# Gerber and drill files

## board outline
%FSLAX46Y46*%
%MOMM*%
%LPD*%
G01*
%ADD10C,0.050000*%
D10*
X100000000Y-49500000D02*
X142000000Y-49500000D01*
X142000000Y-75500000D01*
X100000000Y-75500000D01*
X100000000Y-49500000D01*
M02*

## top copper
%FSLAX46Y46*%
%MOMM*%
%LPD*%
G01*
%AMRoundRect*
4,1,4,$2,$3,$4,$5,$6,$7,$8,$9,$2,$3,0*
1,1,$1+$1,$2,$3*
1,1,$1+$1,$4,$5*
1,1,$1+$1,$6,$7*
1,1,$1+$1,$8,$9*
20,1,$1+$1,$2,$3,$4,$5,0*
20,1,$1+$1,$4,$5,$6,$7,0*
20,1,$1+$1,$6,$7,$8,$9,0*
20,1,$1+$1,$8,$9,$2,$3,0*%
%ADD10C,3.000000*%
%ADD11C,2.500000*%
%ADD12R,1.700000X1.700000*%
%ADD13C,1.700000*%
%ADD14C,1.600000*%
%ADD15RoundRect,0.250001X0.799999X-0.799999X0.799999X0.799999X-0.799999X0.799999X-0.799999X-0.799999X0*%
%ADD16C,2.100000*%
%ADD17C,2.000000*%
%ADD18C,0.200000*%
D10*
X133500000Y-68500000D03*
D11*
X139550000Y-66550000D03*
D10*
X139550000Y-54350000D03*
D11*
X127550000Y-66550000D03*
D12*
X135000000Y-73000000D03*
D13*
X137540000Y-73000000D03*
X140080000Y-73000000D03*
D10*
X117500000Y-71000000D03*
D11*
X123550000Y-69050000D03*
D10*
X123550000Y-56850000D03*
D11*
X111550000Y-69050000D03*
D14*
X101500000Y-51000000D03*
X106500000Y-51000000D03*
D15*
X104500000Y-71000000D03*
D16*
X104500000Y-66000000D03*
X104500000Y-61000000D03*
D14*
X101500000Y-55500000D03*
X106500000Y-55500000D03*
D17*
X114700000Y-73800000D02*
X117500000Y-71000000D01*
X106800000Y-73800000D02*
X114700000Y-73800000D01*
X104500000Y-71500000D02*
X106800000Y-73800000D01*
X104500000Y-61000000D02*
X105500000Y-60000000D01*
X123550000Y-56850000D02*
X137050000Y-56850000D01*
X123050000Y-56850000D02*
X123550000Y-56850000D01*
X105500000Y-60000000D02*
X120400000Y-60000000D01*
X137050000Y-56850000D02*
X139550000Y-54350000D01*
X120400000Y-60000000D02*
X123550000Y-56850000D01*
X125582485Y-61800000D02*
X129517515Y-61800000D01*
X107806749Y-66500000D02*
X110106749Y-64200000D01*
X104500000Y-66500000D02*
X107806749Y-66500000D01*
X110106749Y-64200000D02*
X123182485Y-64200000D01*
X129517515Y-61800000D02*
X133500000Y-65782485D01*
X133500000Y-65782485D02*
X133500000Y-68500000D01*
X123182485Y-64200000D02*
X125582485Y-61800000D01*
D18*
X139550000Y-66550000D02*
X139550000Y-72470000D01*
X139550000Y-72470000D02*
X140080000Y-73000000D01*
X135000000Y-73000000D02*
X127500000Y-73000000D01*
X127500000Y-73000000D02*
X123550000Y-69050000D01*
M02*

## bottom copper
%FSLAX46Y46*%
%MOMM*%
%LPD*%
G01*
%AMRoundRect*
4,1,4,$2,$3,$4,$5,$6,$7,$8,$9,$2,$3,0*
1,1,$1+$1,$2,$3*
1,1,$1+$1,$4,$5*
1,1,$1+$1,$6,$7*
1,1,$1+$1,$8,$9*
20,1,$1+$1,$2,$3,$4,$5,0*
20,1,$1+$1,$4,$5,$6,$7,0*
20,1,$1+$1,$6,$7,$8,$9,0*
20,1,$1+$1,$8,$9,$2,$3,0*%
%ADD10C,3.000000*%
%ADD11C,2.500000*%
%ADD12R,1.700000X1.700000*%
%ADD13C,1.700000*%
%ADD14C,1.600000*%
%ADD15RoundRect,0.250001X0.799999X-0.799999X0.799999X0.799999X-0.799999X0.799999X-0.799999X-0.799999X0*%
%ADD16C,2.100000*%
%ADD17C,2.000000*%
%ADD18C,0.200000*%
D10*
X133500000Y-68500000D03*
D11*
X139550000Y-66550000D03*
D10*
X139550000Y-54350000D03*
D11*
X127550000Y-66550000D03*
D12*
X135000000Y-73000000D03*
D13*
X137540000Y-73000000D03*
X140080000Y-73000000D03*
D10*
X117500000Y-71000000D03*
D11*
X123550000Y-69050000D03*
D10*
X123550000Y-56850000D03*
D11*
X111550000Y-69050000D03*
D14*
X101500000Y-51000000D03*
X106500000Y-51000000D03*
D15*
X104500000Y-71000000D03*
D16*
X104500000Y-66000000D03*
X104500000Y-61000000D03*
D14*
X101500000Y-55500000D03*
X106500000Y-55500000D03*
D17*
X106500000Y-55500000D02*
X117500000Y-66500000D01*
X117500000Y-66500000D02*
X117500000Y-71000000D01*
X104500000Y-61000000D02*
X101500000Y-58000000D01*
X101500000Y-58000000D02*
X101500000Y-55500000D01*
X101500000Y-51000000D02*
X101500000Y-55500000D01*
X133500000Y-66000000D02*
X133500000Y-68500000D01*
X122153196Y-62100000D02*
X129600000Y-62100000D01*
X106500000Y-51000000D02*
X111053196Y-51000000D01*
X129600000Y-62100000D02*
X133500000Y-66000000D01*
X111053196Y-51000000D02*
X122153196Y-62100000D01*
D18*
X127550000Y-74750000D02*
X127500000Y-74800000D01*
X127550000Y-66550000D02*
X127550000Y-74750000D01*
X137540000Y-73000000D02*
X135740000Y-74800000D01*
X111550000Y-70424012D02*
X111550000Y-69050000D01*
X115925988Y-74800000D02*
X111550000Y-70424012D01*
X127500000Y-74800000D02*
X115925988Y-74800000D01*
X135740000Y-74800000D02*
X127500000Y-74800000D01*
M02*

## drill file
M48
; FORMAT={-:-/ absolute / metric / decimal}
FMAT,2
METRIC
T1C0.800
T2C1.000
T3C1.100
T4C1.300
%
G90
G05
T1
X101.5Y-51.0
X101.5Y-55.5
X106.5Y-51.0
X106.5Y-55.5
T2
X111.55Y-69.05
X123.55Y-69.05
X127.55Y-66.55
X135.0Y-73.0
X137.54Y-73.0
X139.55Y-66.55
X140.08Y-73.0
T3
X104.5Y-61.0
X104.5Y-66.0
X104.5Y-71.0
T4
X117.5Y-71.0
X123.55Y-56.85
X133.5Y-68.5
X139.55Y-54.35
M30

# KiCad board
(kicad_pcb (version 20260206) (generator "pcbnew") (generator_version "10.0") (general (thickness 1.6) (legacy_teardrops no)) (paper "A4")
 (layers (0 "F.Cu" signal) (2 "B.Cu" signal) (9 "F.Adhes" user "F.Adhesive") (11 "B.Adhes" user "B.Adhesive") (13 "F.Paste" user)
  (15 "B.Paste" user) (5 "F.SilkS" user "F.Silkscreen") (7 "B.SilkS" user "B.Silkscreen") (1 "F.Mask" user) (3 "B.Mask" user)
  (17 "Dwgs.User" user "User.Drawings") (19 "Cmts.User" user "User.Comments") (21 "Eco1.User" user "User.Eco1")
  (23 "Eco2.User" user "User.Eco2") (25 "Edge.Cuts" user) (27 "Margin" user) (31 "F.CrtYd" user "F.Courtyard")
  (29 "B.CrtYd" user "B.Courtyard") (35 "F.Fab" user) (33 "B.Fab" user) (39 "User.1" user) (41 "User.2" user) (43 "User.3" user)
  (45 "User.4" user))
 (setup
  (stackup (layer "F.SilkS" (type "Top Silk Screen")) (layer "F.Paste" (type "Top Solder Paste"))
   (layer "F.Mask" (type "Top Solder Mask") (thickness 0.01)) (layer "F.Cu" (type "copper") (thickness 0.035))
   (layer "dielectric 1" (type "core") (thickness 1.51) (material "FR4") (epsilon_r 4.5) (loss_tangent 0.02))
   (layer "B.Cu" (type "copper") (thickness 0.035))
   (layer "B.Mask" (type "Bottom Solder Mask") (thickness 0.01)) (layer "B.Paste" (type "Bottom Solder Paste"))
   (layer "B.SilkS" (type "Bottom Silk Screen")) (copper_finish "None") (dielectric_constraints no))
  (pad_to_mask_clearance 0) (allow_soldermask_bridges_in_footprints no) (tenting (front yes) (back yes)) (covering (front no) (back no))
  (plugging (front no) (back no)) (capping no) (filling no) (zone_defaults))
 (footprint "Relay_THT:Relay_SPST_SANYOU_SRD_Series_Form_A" (layer "F.Cu") (at 133.5 68.5 90)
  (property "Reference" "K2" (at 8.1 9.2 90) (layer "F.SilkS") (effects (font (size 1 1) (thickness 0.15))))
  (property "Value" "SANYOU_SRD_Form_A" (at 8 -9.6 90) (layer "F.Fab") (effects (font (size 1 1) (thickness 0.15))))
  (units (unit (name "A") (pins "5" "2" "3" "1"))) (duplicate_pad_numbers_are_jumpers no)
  (pad "1" thru_hole circle (at 0 0 180) (size 3 3) (drill 1.3) (layers "*.Cu" "*.Mask") (remove_unused_layers no) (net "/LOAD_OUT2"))
  (pad "2" thru_hole circle (at 1.95 6.05 180) (size 2.5 2.5) (drill 1) (layers "*.Cu" "*.Mask") (remove_unused_layers no)
   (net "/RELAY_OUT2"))
  (pad "3" thru_hole circle (at 14.15 6.05 180) (size 3 3) (drill 1.3) (layers "*.Cu" "*.Mask") (remove_unused_layers no)
   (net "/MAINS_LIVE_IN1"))
  (pad "5" thru_hole circle (at 1.95 -5.95 180) (size 2.5 2.5) (drill 1) (layers "*.Cu" "*.Mask") (remove_unused_layers no) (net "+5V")))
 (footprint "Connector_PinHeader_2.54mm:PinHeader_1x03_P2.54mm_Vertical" (layer "F.Cu") (at 135 73 90)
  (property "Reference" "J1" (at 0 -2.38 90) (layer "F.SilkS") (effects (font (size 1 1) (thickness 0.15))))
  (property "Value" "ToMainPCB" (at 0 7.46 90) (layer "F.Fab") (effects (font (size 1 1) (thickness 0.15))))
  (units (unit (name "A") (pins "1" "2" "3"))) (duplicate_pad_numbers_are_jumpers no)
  (pad "1" thru_hole rect (at 0 0 90) (size 1.7 1.7) (drill 1) (layers "*.Cu" "*.Mask") (remove_unused_layers no) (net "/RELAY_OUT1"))
  (pad "2" thru_hole circle (at 0 2.54 90) (size 1.7 1.7) (drill 1) (layers "*.Cu" "*.Mask") (remove_unused_layers no) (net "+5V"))
  (pad "3" thru_hole circle (at 0 5.08 90) (size 1.7 1.7) (drill 1) (layers "*.Cu" "*.Mask") (remove_unused_layers no) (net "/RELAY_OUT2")))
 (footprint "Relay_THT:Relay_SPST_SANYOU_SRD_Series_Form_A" (layer "F.Cu") (at 117.5 71 90)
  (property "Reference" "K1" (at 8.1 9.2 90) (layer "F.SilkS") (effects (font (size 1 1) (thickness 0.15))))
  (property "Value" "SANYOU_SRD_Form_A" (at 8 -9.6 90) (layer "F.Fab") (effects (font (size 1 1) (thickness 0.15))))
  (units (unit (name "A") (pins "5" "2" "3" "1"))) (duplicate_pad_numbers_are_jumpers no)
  (pad "1" thru_hole circle (at 0 0 180) (size 3 3) (drill 1.3) (layers "*.Cu" "*.Mask") (remove_unused_layers no) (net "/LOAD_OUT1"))
  (pad "2" thru_hole circle (at 1.95 6.05 180) (size 2.5 2.5) (drill 1) (layers "*.Cu" "*.Mask") (remove_unused_layers no)
   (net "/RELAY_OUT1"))
  (pad "3" thru_hole circle (at 14.15 6.05 180) (size 3 3) (drill 1.3) (layers "*.Cu" "*.Mask") (remove_unused_layers no)
   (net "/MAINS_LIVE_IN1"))
  (pad "5" thru_hole circle (at 1.95 -5.95 180) (size 2.5 2.5) (drill 1) (layers "*.Cu" "*.Mask") (remove_unused_layers no) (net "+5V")))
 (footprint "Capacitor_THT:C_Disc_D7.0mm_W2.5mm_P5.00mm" (layer "F.Cu") (at 101.5 51)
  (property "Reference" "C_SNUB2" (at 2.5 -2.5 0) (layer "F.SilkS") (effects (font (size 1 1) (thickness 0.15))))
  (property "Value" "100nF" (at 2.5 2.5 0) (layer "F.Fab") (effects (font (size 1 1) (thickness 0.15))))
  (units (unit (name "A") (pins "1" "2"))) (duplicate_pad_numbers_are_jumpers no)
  (pad "1" thru_hole circle (at 0 0) (size 1.6 1.6) (drill 0.8) (layers "*.Cu" "*.Mask") (remove_unused_layers no) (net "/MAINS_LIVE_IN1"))
  (pad "2" thru_hole circle (at 5 0) (size 1.6 1.6) (drill 0.8) (layers "*.Cu" "*.Mask") (remove_unused_layers no) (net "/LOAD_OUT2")))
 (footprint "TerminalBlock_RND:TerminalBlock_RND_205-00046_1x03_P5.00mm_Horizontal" (layer "F.Cu") (at 104.5 71 90)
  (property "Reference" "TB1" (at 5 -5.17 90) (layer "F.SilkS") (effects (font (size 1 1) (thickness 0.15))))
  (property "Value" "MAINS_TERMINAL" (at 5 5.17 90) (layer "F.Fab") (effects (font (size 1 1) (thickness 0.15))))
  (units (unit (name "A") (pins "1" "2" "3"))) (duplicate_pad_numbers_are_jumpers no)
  (pad "1" thru_hole roundrect (at 0 0 90) (size 2.1 2.1) (drill 1.1) (layers "*.Cu" "*.Mask") (remove_unused_layers no)
   (roundrect_rratio 0.119048) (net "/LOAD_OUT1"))
  (pad "2" thru_hole circle (at 5 0 90) (size 2.1 2.1) (drill 1.1) (layers "*.Cu" "*.Mask") (remove_unused_layers no) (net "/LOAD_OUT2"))
  (pad "3" thru_hole circle (at 10 0 90) (size 2.1 2.1) (drill 1.1) (layers "*.Cu" "*.Mask") (remove_unused_layers no)
   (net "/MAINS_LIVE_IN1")))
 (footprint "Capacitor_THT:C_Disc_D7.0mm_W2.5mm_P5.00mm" (layer "F.Cu") (at 101.5 55.5)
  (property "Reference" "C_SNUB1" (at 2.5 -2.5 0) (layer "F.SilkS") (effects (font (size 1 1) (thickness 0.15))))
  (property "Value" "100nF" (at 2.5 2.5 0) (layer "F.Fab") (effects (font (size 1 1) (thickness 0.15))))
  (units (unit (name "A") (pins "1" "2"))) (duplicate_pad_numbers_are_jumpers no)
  (pad "1" thru_hole circle (at 0 0) (size 1.6 1.6) (drill 0.8) (layers "*.Cu" "*.Mask") (remove_unused_layers no) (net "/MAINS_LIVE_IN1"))
  (pad "2" thru_hole circle (at 5 0) (size 1.6 1.6) (drill 0.8) (layers "*.Cu" "*.Mask") (remove_unused_layers no) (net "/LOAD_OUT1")))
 (gr_rect (start 100 49.5) (end 142 75.5) (stroke (width 0.05) (type default)) (fill no) (layer "Edge.Cuts"))
 (segment (start 114.7 73.8) (end 117.5 71) (width 2) (layer "F.Cu") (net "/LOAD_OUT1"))
 (segment (start 106.8 73.8) (end 114.7 73.8) (width 2) (layer "F.Cu") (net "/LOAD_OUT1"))
 (segment (start 104.5 71.5) (end 106.8 73.8) (width 2) (layer "F.Cu") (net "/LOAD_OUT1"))
 (segment (start 106.5 55.5) (end 117.5 66.5) (width 2) (layer "B.Cu") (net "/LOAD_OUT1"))
 (segment (start 117.5 66.5) (end 117.5 71) (width 2) (layer "B.Cu") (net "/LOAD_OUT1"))
 (segment (start 104.5 61) (end 105.5 60) (width 2) (layer "F.Cu") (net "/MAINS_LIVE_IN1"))
 (segment (start 123.55 56.85) (end 137.05 56.85) (width 2) (layer "F.Cu") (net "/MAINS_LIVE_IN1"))
 (segment (start 123.05 56.85) (end 123.55 56.85) (width 2) (layer "F.Cu") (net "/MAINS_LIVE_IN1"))
 (segment (start 105.5 60) (end 120.4 60) (width 2) (layer "F.Cu") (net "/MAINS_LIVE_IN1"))
 (segment (start 137.05 56.85) (end 139.55 54.35) (width 2) (layer "F.Cu") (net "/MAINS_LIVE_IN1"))
 (segment (start 120.4 60) (end 123.55 56.85) (width 2) (layer "F.Cu") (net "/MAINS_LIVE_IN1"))
 (segment (start 104.5 61) (end 101.5 58) (width 2) (layer "B.Cu") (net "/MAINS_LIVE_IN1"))
 (segment (start 101.5 58) (end 101.5 55.5) (width 2) (layer "B.Cu") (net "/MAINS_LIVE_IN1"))
 (segment (start 101.5 51) (end 101.5 55.5) (width 2) (layer "B.Cu") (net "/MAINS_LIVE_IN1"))
 (segment (start 125.582485 61.8) (end 129.517515 61.8) (width 2) (layer "F.Cu") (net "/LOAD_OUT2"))
 (segment (start 107.806749 66.5) (end 110.106749 64.2) (width 2) (layer "F.Cu") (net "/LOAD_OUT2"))
 (segment (start 104.5 66.5) (end 107.806749 66.5) (width 2) (layer "F.Cu") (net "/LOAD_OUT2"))
 (segment (start 110.106749 64.2) (end 123.182485 64.2) (width 2) (layer "F.Cu") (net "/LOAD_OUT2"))
 (segment (start 129.517515 61.8) (end 133.5 65.782485) (width 2) (layer "F.Cu") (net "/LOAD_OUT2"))
 (segment (start 133.5 65.782485) (end 133.5 68.5) (width 2) (layer "F.Cu") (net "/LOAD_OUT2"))
 (segment (start 123.182485 64.2) (end 125.582485 61.8) (width 2) (layer "F.Cu") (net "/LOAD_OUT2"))
 (segment (start 133.5 66) (end 133.5 68.5) (width 2) (layer "B.Cu") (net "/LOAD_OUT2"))
 (segment (start 122.153196 62.1) (end 129.6 62.1) (width 2) (layer "B.Cu") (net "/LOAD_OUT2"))
 (segment (start 106.5 51) (end 111.053196 51) (width 2) (layer "B.Cu") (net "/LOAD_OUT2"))
 (segment (start 129.6 62.1) (end 133.5 66) (width 2) (layer "B.Cu") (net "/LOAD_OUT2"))
 (segment (start 111.053196 51) (end 122.153196 62.1) (width 2) (layer "B.Cu") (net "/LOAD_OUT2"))
 (segment (start 139.55 66.55) (end 139.55 72.47) (width 0.2) (layer "F.Cu") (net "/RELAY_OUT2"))
 (segment (start 139.55 72.47) (end 140.08 73) (width 0.2) (layer "F.Cu") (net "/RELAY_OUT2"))
 (segment (start 135 73) (end 127.5 73) (width 0.2) (layer "F.Cu") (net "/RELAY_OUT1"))
 (segment (start 127.5 73) (end 123.55 69.05) (width 0.2) (layer "F.Cu") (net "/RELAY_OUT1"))
 (segment (start 127.55 74.75) (end 127.5 74.8) (width 0.2) (layer "B.Cu") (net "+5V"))
 (segment (start 127.55 66.55) (end 127.55 74.75) (width 0.2) (layer "B.Cu") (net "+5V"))
 (segment (start 137.54 73) (end 135.74 74.8) (width 0.2) (layer "B.Cu") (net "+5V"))
 (segment (start 111.55 70.424012) (end 111.55 69.05) (width 0.2) (layer "B.Cu") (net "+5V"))
 (segment (start 115.925988 74.8) (end 111.55 70.424012) (width 0.2) (layer "B.Cu") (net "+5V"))
 (segment (start 127.5 74.8) (end 115.925988 74.8) (width 0.2) (layer "B.Cu") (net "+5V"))
 (segment (start 135.74 74.8) (end 127.5 74.8) (width 0.2) (layer "B.Cu") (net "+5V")))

